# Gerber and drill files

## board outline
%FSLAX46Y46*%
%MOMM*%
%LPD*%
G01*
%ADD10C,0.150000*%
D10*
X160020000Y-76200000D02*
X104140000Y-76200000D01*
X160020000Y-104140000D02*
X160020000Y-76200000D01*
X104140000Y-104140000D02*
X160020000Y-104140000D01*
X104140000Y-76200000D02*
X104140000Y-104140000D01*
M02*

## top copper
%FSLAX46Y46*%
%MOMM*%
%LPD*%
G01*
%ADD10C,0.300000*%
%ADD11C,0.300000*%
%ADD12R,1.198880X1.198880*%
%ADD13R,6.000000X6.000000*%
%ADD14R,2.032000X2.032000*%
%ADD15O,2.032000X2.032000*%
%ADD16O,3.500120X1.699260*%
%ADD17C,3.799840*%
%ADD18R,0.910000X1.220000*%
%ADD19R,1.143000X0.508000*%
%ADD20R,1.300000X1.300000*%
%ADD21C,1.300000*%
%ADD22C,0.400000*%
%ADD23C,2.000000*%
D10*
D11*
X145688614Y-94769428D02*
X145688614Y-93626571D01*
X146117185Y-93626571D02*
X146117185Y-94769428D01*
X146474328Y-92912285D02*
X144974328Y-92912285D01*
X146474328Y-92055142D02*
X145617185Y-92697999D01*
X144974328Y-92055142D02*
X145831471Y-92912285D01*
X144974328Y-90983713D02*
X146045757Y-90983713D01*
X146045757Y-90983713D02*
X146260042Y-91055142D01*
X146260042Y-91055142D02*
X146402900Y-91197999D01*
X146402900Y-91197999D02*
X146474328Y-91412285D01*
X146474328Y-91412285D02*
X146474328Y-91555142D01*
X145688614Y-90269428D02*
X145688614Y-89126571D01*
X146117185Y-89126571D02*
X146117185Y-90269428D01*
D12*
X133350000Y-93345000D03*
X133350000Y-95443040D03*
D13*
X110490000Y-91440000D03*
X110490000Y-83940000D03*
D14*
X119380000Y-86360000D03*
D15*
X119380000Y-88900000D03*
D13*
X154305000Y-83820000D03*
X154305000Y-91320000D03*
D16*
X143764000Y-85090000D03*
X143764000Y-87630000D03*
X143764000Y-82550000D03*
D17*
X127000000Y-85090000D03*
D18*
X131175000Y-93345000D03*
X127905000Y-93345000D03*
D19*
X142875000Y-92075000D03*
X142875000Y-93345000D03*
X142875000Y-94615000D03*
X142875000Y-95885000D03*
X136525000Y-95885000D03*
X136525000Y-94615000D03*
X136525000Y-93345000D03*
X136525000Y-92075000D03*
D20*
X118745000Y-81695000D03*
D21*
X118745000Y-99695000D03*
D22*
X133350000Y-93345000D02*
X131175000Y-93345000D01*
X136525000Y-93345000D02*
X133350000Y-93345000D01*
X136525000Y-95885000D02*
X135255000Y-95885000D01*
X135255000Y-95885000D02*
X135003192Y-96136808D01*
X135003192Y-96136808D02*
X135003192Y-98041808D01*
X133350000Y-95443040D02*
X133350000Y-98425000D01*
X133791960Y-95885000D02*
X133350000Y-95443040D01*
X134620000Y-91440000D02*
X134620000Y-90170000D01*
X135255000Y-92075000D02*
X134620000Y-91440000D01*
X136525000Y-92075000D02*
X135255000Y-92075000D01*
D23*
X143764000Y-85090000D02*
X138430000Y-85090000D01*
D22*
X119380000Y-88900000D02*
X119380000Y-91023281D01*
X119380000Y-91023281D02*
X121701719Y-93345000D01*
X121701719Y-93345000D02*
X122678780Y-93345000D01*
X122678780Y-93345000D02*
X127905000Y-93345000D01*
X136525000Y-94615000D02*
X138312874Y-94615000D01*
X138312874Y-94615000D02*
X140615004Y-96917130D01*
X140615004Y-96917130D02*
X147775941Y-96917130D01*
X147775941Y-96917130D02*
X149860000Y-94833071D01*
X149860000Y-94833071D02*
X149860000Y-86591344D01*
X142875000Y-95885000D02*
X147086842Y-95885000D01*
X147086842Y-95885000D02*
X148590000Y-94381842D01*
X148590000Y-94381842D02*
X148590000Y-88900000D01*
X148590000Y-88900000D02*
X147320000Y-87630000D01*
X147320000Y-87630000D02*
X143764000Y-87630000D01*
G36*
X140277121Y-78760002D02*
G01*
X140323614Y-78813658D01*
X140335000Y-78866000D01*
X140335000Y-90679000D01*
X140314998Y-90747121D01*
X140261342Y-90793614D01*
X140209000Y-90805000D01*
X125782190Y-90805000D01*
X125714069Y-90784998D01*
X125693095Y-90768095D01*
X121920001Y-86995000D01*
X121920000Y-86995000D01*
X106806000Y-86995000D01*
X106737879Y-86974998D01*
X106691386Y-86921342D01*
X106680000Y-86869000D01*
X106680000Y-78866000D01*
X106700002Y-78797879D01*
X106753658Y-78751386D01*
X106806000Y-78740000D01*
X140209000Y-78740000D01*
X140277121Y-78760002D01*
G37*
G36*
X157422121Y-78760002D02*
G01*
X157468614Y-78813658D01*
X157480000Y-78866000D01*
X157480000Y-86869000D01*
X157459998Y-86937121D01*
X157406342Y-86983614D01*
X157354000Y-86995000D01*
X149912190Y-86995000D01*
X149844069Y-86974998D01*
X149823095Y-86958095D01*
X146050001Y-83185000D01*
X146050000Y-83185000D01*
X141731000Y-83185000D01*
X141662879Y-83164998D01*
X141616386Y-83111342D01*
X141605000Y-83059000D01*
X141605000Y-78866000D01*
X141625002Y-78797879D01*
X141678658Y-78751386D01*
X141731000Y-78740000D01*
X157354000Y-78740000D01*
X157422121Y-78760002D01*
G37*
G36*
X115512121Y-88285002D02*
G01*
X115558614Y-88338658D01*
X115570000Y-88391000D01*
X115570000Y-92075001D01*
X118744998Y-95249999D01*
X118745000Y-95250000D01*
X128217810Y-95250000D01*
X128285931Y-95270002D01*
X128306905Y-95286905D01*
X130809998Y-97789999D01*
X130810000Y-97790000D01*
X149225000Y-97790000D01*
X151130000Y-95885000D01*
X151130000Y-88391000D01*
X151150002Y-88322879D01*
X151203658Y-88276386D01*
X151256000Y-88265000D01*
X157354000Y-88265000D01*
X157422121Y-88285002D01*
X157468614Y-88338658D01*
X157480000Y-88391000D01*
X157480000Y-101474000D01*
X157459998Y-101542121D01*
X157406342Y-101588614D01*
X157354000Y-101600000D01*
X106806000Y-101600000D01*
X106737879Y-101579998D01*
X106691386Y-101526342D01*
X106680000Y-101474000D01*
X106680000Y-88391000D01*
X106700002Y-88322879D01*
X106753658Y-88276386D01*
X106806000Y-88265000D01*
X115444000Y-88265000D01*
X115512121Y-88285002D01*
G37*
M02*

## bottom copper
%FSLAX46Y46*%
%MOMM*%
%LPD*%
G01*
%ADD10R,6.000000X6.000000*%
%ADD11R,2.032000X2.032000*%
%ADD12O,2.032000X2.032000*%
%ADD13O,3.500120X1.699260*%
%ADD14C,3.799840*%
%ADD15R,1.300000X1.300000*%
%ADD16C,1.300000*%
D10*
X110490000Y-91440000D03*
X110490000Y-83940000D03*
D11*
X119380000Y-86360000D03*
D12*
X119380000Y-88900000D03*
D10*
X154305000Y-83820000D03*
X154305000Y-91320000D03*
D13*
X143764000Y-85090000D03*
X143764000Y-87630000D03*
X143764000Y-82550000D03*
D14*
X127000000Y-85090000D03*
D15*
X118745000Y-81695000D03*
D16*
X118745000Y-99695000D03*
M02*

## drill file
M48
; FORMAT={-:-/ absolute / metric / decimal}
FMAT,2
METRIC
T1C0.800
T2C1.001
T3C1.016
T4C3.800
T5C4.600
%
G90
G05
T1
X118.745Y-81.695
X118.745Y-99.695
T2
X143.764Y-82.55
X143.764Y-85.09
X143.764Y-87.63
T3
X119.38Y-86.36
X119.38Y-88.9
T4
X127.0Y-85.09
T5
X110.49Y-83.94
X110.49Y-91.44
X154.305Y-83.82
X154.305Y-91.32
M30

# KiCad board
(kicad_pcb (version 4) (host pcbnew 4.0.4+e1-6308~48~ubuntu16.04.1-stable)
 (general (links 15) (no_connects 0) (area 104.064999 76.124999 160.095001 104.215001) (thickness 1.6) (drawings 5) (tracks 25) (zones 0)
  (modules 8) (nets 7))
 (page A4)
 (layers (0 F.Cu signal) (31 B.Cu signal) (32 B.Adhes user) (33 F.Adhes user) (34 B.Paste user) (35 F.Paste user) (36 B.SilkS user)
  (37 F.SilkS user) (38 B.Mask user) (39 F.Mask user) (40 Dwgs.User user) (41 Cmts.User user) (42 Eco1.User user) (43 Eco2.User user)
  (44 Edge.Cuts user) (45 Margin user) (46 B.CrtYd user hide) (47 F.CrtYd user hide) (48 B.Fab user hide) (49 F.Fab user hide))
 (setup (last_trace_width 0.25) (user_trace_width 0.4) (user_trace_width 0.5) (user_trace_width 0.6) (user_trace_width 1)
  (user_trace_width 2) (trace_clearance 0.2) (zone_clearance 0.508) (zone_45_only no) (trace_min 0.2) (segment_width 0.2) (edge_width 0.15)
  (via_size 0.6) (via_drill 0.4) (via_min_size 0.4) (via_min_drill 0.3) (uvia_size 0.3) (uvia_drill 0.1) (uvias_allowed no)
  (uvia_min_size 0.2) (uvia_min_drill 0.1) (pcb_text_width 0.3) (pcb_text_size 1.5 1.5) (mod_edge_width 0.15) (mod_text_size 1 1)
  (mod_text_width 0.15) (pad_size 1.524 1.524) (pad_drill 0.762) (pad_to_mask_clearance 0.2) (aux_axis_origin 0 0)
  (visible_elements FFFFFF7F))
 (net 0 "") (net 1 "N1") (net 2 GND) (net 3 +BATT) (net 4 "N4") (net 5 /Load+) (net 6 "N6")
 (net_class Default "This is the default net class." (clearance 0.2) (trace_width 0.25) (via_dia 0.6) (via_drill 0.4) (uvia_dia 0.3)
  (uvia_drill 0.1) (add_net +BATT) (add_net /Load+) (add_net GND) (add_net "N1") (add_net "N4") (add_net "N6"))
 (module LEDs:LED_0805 (layer F.Cu) (at 133.35 94.39402 90)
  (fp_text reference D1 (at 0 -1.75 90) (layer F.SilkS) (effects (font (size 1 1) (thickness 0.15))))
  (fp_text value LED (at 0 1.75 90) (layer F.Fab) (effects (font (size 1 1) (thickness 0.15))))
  (pad 2 smd rect (at 1.04902 0 270) (size 1.19888 1.19888) (layers F.Cu F.Paste F.Mask) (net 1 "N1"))
  (pad 1 smd rect (at -1.04902 0 270) (size 1.19888 1.19888) (layers F.Cu F.Paste F.Mask) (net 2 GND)))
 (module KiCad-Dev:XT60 (layer B.Cu) (at 110.49 91.44 90)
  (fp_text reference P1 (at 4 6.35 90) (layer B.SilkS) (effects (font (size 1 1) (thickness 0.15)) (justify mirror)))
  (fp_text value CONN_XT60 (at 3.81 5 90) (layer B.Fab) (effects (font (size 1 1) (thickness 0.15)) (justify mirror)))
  (pad 1 thru_hole rect (at 0 0 90) (size 6 6) (drill 4.6) (layers *.Cu *.Mask) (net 2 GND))
  (pad 2 thru_hole rect (at 7.5 0 90) (size 6 6) (drill 4.6) (layers *.Cu *.Mask) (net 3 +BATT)))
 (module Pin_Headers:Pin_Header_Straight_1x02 (layer B.Cu) (at 119.38 86.36 180)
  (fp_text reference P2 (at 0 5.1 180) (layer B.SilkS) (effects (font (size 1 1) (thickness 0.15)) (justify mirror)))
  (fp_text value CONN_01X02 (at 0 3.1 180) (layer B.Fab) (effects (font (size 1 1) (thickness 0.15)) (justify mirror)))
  (pad 1 thru_hole rect (at 0 0 180) (size 2.032 2.032) (drill 1.016) (layers *.Cu *.Mask B.SilkS) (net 3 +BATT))
  (pad 2 thru_hole oval (at 0 -2.54 180) (size 2.032 2.032) (drill 1.016) (layers *.Cu *.Mask B.SilkS) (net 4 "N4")))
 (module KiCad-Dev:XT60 (layer B.Cu) (at 154.305 83.82 270)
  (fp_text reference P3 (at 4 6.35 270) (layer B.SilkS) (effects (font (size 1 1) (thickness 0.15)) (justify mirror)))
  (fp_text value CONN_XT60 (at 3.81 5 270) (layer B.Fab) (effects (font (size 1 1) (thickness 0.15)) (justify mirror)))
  (pad 1 thru_hole rect (at 0 0 270) (size 6 6) (drill 4.6) (layers *.Cu *.Mask) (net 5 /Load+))
  (pad 2 thru_hole rect (at 7.5 0 270) (size 6 6) (drill 4.6) (layers *.Cu *.Mask) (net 2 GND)))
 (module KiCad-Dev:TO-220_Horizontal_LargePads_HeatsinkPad (layer F.Cu) (at 143.764 85.09 90)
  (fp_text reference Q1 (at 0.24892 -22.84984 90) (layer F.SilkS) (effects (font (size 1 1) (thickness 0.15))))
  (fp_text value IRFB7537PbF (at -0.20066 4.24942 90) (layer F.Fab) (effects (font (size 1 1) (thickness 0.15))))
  (pad 2 thru_hole oval (at 0 0 180) (size 3.50012 1.69926) (drill 1.00076) (layers *.Cu *.Mask F.SilkS) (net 3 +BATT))
  (pad 1 thru_hole oval (at -2.54 0 180) (size 3.50012 1.69926) (drill 1.00076) (layers *.Cu *.Mask F.SilkS) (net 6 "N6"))
  (pad 3 thru_hole oval (at 2.54 0 180) (size 3.50012 1.69926) (drill 1.00076) (layers *.Cu *.Mask F.SilkS) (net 5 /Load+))
  (pad 2 thru_hole circle (at 0 -16.764 180) (size 3.79984 3.79984) (drill 3.79984) (layers *.Cu *.Mask) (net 3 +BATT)))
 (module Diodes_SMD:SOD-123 (layer F.Cu) (at 129.54 93.345 180)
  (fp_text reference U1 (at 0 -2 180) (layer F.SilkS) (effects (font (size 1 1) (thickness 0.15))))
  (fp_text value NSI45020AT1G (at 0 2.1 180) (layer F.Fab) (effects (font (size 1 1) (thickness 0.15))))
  (pad 1 smd rect (at -1.635 0 180) (size 0.91 1.22) (layers F.Cu F.Paste F.Mask) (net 1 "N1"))
  (pad 2 smd rect (at 1.635 0 180) (size 0.91 1.22) (layers F.Cu F.Paste F.Mask) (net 4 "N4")))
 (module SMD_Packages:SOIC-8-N (layer F.Cu) (at 139.7 93.98 270)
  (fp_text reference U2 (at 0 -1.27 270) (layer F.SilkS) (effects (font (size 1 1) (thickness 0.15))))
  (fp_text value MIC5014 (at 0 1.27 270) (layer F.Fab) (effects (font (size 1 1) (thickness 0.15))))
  (pad 8 smd rect (at -1.905 -3.175 270) (size 0.508 1.143) (layers F.Cu F.Paste F.Mask))
  (pad 7 smd rect (at -0.635 -3.175 270) (size 0.508 1.143) (layers F.Cu F.Paste F.Mask))
  (pad 6 smd rect (at 0.635 -3.175 270) (size 0.508 1.143) (layers F.Cu F.Paste F.Mask))
  (pad 5 smd rect (at 1.905 -3.175 270) (size 0.508 1.143) (layers F.Cu F.Paste F.Mask) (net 6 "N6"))
  (pad 4 smd rect (at 1.905 3.175 270) (size 0.508 1.143) (layers F.Cu F.Paste F.Mask) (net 2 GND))
  (pad 3 smd rect (at 0.635 3.175 270) (size 0.508 1.143) (layers F.Cu F.Paste F.Mask) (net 5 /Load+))
  (pad 2 smd rect (at -0.635 3.175 270) (size 0.508 1.143) (layers F.Cu F.Paste F.Mask) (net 1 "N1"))
  (pad 1 smd rect (at -1.905 3.175 270) (size 0.508 1.143) (layers F.Cu F.Paste F.Mask) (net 3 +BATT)))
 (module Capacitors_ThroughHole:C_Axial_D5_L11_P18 (layer F.Cu) (at 118.745 81.695 270)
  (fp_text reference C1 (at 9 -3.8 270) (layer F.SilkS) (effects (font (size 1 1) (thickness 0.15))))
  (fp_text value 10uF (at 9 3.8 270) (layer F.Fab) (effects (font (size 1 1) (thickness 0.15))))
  (pad 1 thru_hole rect (at 0 0 270) (size 1.3 1.3) (drill 0.8) (layers *.Cu *.Mask F.SilkS) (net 3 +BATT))
  (pad 2 thru_hole circle (at 18 0 270) (size 1.3 1.3) (drill 0.8) (layers *.Cu *.Mask F.SilkS) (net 2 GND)))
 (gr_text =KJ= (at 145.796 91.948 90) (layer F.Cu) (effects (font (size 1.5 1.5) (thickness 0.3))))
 (gr_line (start 160.02 76.2) (end 104.14 76.2) (layer Edge.Cuts) (width 0.15))
 (gr_line (start 160.02 104.14) (end 160.02 76.2) (layer Edge.Cuts) (width 0.15))
 (gr_line (start 104.14 104.14) (end 160.02 104.14) (layer Edge.Cuts) (width 0.15))
 (gr_line (start 104.14 76.2) (end 104.14 104.14) (layer Edge.Cuts) (width 0.15))
 (segment (start 133.35 93.345) (end 131.175 93.345) (width 0.4) (layer F.Cu) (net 1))
 (segment (start 136.525 93.345) (end 133.35 93.345) (width 0.4) (layer F.Cu) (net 1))
 (segment (start 136.525 95.885) (end 135.255 95.885) (width 0.4) (layer F.Cu) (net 2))
 (segment (start 135.255 95.885) (end 135.003192 96.136808) (width 0.4) (layer F.Cu) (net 2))
 (segment (start 135.003192 96.136808) (end 135.003192 98.041808) (width 0.4) (layer F.Cu) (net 2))
 (segment (start 133.35 95.44304) (end 133.35 98.425) (width 0.4) (layer F.Cu) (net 2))
 (segment (start 133.79196 95.885) (end 133.35 95.44304) (width 0.4) (layer F.Cu) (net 2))
 (segment (start 134.62 91.44) (end 134.62 90.17) (width 0.4) (layer F.Cu) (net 3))
 (segment (start 135.255 92.075) (end 134.62 91.44) (width 0.4) (layer F.Cu) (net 3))
 (segment (start 136.525 92.075) (end 135.255 92.075) (width 0.4) (layer F.Cu) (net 3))
 (segment (start 143.764 85.09) (end 138.43 85.09) (width 2) (layer F.Cu) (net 3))
 (segment (start 119.38 88.9) (end 119.38 91.023281) (width 0.4) (layer F.Cu) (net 4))
 (segment (start 119.38 91.023281) (end 121.701719 93.345) (width 0.4) (layer F.Cu) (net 4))
 (segment (start 121.701719 93.345) (end 122.67878 93.345) (width 0.4) (layer F.Cu) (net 4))
 (segment (start 122.67878 93.345) (end 127.905 93.345) (width 0.4) (layer F.Cu) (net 4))
 (segment (start 136.525 94.615) (end 138.312874 94.615) (width 0.4) (layer F.Cu) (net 5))
 (segment (start 138.312874 94.615) (end 140.615004 96.91713) (width 0.4) (layer F.Cu) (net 5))
 (segment (start 140.615004 96.91713) (end 147.775941 96.91713) (width 0.4) (layer F.Cu) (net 5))
 (segment (start 147.775941 96.91713) (end 149.86 94.833071) (width 0.4) (layer F.Cu) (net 5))
 (segment (start 149.86 94.833071) (end 149.86 86.591344) (width 0.4) (layer F.Cu) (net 5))
 (segment (start 142.875 95.885) (end 147.086842 95.885) (width 0.4) (layer F.Cu) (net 6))
 (segment (start 147.086842 95.885) (end 148.59 94.381842) (width 0.4) (layer F.Cu) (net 6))
 (segment (start 148.59 94.381842) (end 148.59 88.9) (width 0.4) (layer F.Cu) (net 6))
 (segment (start 148.59 88.9) (end 147.32 87.63) (width 0.4) (layer F.Cu) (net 6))
 (segment (start 147.32 87.63) (end 143.764 87.63) (width 0.4) (layer F.Cu) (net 6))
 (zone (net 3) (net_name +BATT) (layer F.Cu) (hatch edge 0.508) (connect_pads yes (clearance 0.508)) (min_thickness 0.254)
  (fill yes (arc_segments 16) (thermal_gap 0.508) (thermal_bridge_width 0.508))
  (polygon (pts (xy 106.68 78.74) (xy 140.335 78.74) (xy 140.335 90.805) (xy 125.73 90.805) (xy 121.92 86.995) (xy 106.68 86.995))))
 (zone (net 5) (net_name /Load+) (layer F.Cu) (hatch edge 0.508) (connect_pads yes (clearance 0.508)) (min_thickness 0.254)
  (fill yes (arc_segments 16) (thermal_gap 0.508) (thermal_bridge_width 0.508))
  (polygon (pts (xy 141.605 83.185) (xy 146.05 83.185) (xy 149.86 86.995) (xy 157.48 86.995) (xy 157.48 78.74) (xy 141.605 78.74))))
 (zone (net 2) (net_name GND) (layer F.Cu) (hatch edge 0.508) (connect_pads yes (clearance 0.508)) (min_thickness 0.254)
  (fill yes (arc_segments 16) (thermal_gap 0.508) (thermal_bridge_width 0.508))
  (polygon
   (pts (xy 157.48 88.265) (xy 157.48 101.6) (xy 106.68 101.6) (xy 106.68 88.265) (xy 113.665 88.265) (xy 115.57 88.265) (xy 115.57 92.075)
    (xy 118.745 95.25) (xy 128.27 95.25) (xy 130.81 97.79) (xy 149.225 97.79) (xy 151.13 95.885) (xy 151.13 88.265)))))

